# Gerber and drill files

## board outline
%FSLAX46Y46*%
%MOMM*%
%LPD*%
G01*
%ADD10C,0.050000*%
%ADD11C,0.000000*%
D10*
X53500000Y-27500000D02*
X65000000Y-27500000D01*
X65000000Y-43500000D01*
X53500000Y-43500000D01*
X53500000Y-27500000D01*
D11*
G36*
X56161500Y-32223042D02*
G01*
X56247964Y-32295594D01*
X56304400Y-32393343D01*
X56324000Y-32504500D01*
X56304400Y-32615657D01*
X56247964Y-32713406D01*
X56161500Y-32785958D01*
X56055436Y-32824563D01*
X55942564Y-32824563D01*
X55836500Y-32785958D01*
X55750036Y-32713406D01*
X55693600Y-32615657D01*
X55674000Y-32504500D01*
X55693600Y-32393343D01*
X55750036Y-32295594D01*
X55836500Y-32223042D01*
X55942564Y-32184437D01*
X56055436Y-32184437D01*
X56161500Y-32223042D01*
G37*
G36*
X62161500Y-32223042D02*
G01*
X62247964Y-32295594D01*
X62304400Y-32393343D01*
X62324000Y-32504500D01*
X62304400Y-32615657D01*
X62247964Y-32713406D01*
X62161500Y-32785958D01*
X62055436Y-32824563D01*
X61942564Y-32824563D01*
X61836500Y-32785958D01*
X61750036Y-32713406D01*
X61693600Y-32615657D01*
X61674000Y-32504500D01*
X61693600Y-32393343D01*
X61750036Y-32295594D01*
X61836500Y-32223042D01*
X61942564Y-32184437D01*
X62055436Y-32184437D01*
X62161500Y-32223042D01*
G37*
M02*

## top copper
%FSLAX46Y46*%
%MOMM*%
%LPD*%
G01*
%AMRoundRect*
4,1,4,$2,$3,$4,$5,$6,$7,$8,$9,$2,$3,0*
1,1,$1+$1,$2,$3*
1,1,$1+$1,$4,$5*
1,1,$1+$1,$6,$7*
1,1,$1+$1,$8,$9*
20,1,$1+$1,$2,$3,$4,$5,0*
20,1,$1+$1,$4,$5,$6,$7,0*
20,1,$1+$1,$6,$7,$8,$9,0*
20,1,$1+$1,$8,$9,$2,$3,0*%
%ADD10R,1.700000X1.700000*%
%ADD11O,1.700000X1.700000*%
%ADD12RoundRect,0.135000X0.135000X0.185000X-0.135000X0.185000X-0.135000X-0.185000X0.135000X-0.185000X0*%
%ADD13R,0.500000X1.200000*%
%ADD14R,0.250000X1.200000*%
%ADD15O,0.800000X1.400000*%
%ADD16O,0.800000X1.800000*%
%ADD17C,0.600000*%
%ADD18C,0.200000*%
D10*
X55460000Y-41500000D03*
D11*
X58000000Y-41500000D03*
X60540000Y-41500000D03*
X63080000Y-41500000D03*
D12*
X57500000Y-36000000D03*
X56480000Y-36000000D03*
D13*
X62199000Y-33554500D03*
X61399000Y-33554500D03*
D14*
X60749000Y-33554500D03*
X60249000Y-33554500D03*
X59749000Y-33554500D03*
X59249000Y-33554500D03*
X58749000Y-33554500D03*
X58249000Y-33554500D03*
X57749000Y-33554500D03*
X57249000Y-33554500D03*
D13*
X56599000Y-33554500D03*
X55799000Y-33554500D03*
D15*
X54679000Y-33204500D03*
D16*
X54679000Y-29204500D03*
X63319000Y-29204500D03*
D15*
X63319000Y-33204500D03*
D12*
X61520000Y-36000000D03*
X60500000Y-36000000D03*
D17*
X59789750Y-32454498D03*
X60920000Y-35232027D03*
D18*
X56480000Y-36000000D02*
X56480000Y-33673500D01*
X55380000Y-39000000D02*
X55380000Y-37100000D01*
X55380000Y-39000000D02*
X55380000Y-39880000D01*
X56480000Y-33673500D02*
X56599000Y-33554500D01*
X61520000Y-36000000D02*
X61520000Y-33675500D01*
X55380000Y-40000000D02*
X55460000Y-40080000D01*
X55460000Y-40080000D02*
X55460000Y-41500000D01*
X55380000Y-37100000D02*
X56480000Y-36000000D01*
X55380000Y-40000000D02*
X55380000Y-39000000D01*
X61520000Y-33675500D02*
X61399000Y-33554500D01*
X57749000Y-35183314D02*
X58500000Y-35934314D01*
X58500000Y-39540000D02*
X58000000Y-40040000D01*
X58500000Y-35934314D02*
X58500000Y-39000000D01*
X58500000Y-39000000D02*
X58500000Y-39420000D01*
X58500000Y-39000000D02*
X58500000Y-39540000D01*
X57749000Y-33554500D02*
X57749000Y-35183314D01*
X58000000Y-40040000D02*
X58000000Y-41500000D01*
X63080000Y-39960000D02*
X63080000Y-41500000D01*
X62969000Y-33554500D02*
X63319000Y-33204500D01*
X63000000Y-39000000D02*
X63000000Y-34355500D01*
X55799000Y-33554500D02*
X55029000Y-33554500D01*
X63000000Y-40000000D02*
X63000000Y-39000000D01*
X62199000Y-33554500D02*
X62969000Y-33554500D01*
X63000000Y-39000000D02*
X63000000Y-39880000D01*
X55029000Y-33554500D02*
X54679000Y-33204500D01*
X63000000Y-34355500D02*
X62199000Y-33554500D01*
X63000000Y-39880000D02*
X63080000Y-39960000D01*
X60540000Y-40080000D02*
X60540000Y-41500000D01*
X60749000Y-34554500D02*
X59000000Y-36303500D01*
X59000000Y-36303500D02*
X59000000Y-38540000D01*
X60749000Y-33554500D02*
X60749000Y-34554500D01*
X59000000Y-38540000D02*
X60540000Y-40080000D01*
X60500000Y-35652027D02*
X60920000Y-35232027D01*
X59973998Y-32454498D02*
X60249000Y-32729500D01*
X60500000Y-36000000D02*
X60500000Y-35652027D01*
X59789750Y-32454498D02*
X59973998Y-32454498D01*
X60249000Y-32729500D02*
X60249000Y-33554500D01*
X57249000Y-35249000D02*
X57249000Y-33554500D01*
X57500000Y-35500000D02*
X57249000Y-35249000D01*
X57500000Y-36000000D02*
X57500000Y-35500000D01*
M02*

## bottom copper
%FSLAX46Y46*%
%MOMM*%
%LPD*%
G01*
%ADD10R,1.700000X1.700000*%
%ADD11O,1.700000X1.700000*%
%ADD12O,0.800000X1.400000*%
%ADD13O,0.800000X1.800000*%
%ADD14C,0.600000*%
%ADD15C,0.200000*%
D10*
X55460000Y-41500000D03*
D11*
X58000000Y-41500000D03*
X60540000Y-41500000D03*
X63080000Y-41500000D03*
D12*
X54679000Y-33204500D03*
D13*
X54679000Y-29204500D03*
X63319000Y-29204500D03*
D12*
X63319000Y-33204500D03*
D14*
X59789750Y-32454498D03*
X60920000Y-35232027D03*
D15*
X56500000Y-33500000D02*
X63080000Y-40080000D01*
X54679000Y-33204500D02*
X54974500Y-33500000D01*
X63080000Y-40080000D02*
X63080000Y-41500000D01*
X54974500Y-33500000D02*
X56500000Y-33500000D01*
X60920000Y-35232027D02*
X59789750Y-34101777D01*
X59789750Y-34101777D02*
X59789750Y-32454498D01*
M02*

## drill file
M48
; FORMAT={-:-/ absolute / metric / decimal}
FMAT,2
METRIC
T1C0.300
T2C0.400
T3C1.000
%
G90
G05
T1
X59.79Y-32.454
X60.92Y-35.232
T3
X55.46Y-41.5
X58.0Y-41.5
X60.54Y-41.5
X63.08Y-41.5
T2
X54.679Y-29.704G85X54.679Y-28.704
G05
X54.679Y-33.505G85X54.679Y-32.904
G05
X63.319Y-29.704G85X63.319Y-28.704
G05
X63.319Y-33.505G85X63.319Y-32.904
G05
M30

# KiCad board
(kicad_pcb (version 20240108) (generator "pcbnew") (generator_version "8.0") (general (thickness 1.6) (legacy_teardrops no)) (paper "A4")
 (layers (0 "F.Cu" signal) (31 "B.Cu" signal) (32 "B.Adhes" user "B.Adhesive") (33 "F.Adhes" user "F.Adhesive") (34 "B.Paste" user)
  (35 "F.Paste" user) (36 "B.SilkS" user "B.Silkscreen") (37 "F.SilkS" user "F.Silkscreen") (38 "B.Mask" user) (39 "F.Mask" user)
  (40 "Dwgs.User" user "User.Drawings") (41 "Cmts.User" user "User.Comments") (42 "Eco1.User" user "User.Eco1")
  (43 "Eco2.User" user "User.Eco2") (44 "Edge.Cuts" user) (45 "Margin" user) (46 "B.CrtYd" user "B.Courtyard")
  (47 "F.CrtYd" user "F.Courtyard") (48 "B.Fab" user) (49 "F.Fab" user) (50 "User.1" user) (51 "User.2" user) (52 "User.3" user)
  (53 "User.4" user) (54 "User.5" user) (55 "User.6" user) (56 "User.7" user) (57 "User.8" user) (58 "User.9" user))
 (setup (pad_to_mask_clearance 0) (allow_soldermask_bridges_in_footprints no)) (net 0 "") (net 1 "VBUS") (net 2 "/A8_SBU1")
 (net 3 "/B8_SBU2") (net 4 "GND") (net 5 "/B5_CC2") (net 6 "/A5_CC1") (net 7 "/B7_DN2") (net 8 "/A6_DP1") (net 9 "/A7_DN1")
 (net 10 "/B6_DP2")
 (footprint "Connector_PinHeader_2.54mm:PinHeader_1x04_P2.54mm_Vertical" (layer "F.Cu") (at 55.46 41.5 90)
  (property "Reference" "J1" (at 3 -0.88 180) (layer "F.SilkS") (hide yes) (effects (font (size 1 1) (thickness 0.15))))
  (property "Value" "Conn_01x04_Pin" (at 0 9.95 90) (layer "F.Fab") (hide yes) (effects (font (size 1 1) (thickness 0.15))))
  (pad "1" thru_hole rect (at 0 0 90) (size 1.7 1.7) (drill 1) (layers "*.Cu" "*.Mask") (remove_unused_layers no) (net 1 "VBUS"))
  (pad "2" thru_hole oval (at 0 2.54 90) (size 1.7 1.7) (drill 1) (layers "*.Cu" "*.Mask") (remove_unused_layers no) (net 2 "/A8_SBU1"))
  (pad "3" thru_hole oval (at 0 5.08 90) (size 1.7 1.7) (drill 1) (layers "*.Cu" "*.Mask") (remove_unused_layers no) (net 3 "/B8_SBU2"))
  (pad "4" thru_hole oval (at 0 7.62 90) (size 1.7 1.7) (drill 1) (layers "*.Cu" "*.Mask") (remove_unused_layers no) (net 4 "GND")))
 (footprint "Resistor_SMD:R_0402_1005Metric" (layer "F.Cu") (at 56.99 36 180)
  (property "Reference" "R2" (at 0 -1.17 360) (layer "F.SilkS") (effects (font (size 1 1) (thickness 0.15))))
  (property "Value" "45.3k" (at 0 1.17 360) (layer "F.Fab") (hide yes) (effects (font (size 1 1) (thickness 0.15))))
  (pad "1" smd roundrect (at -0.51 0 180) (size 0.54 0.64) (layers "F.Cu" "F.Paste" "F.Mask") (roundrect_rratio 0.25) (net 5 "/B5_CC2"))
  (pad "2" smd roundrect (at 0.51 0 180) (size 0.54 0.64) (layers "F.Cu" "F.Paste" "F.Mask") (roundrect_rratio 0.25) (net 1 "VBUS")))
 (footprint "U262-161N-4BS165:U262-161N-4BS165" (layer "F.Cu") (at 58.999 31.3795 180)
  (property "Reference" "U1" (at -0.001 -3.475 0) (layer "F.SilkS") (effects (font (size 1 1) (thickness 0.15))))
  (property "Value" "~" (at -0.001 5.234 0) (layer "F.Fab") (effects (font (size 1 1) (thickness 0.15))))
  (fp_poly
   (pts (xy 3.325 -1.125) (xy 3.3054 -1.236157) (xy 3.248964 -1.333906) (xy 3.1625 -1.406458) (xy 3.056436 -1.445063)
    (xy 2.943564 -1.445063) (xy 2.8375 -1.406458) (xy 2.751036 -1.333906) (xy 2.6946 -1.236157) (xy 2.675 -1.125) (xy 2.6946 -1.013843)
    (xy 2.751036 -0.916094) (xy 2.8375 -0.843542) (xy 2.943564 -0.804937) (xy 3.056436 -0.804937) (xy 3.1625 -0.843542)
    (xy 3.248964 -0.916094) (xy 3.3054 -1.013843))
   (stroke (width 0) (type default)) (fill solid) (layer "Edge.Cuts"))
  (fp_poly
   (pts (xy -2.675 -1.125) (xy -2.6946 -1.236157) (xy -2.751036 -1.333906) (xy -2.8375 -1.406458) (xy -2.943564 -1.445063)
    (xy -3.056436 -1.445063) (xy -3.1625 -1.406458) (xy -3.248964 -1.333906) (xy -3.3054 -1.236157) (xy -3.325 -1.125)
    (xy -3.3054 -1.013843) (xy -3.248964 -0.916094) (xy -3.1625 -0.843542) (xy -3.056436 -0.804937) (xy -2.943564 -0.804937)
    (xy -2.8375 -0.843542) (xy -2.751036 -0.916094) (xy -2.6946 -1.013843))
   (stroke (width 0) (type default)) (fill solid) (layer "Edge.Cuts"))
  (pad "1" smd rect (at -3.2 -2.175 180) (size 0.5 1.2) (layers "F.Cu" "F.Paste" "F.Mask") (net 4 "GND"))
  (pad "2" smd rect (at -2.4 -2.175 180) (size 0.5 1.2) (layers "F.Cu" "F.Paste" "F.Mask") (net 1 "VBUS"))
  (pad "3" smd rect (at -1.75 -2.175 180) (size 0.25 1.2) (layers "F.Cu" "F.Paste" "F.Mask") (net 3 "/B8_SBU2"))
  (pad "4" smd rect (at -1.25 -2.175 180) (size 0.25 1.2) (layers "F.Cu" "F.Paste" "F.Mask") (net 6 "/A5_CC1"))
  (pad "5" smd rect (at -0.75 -2.175 180) (size 0.25 1.2) (layers "F.Cu" "F.Paste" "F.Mask") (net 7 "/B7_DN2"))
  (pad "6" smd rect (at -0.25 -2.175 180) (size 0.25 1.2) (layers "F.Cu" "F.Paste" "F.Mask") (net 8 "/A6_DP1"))
  (pad "7" smd rect (at 0.25 -2.175 180) (size 0.25 1.2) (layers "F.Cu" "F.Paste" "F.Mask") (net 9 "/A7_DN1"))
  (pad "8" smd rect (at 0.75 -2.175 180) (size 0.25 1.2) (layers "F.Cu" "F.Paste" "F.Mask") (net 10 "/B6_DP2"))
  (pad "9" smd rect (at 1.25 -2.175 180) (size 0.25 1.2) (layers "F.Cu" "F.Paste" "F.Mask") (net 2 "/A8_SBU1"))
  (pad "10" smd rect (at 1.75 -2.175 180) (size 0.25 1.2) (layers "F.Cu" "F.Paste" "F.Mask") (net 5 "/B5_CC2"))
  (pad "11" smd rect (at 2.4 -2.175 180) (size 0.5 1.2) (layers "F.Cu" "F.Paste" "F.Mask") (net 1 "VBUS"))
  (pad "12" smd rect (at 3.2 -2.175 180) (size 0.5 1.2) (layers "F.Cu" "F.Paste" "F.Mask") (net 4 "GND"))
  (pad "13" thru_hole oval (at 4.32 -1.825 180) (size 0.8 1.4) (drill oval 0.4 1) (layers "*.Cu" "*.Mask") (remove_unused_layers no)
   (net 4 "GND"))
  (pad "14" thru_hole oval (at 4.32 2.175 180) (size 0.8 1.8) (drill oval 0.4 1.4) (layers "*.Cu" "*.Mask") (remove_unused_layers no)
   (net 4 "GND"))
  (pad "15" thru_hole oval (at -4.32 2.175 180) (size 0.8 1.8) (drill oval 0.4 1.4) (layers "*.Cu" "*.Mask") (remove_unused_layers no)
   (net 4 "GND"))
  (pad "16" thru_hole oval (at -4.32 -1.825 180) (size 0.8 1.4) (drill oval 0.4 1) (layers "*.Cu" "*.Mask") (remove_unused_layers no)
   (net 4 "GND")))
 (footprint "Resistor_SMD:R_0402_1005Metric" (layer "F.Cu") (at 61.01 36 180)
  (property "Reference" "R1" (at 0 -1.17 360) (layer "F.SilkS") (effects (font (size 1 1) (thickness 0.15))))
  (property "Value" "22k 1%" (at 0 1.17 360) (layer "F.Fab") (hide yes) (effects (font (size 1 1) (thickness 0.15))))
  (pad "1" smd roundrect (at -0.51 0 180) (size 0.54 0.64) (layers "F.Cu" "F.Paste" "F.Mask") (roundrect_rratio 0.25) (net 1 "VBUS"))
  (pad "2" smd roundrect (at 0.51 0 180) (size 0.54 0.64) (layers "F.Cu" "F.Paste" "F.Mask") (roundrect_rratio 0.25) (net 6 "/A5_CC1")))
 (gr_rect (start 53.5 27.5) (end 65 43.5) (stroke (width 0.05) (type default)) (fill none) (layer "Edge.Cuts"))
 (segment (start 56.48 36) (end 56.48 33.6735) (width 0.2) (layer "F.Cu") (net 1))
 (segment (start 55.38 39) (end 55.38 37.1) (width 0.2) (layer "F.Cu") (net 1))
 (segment (start 55.38 39) (end 55.38 39.88) (width 0.2) (layer "F.Cu") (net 1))
 (segment (start 56.48 33.6735) (end 56.599 33.5545) (width 0.2) (layer "F.Cu") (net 1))
 (segment (start 61.52 36) (end 61.52 33.6755) (width 0.2) (layer "F.Cu") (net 1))
 (segment (start 55.38 40) (end 55.46 40.08) (width 0.2) (layer "F.Cu") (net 1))
 (segment (start 55.46 40.08) (end 55.46 41.5) (width 0.2) (layer "F.Cu") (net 1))
 (segment (start 55.38 37.1) (end 56.48 36) (width 0.2) (layer "F.Cu") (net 1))
 (segment (start 55.38 40) (end 55.38 39) (width 0.2) (layer "F.Cu") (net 1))
 (segment (start 61.52 33.6755) (end 61.399 33.5545) (width 0.2) (layer "F.Cu") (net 1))
 (segment (start 57.749 35.183314) (end 58.5 35.934314) (width 0.2) (layer "F.Cu") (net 2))
 (segment (start 58.5 39.54) (end 58 40.04) (width 0.2) (layer "F.Cu") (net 2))
 (segment (start 58.5 35.934314) (end 58.5 39) (width 0.2) (layer "F.Cu") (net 2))
 (segment (start 58.5 39) (end 58.5 39.42) (width 0.2) (layer "F.Cu") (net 2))
 (segment (start 58.5 39) (end 58.5 39.54) (width 0.2) (layer "F.Cu") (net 2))
 (segment (start 57.749 33.5545) (end 57.749 35.183314) (width 0.2) (layer "F.Cu") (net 2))
 (segment (start 58 40.04) (end 58 41.5) (width 0.2) (layer "F.Cu") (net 2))
 (segment (start 63.08 39.96) (end 63.08 41.5) (width 0.2) (layer "F.Cu") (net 4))
 (segment (start 62.969 33.5545) (end 63.319 33.2045) (width 0.2) (layer "F.Cu") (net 4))
 (segment (start 63 39) (end 63 34.3555) (width 0.2) (layer "F.Cu") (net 4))
 (segment (start 55.799 33.5545) (end 55.029 33.5545) (width 0.2) (layer "F.Cu") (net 4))
 (segment (start 63 40) (end 63 39) (width 0.2) (layer "F.Cu") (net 4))
 (segment (start 62.199 33.5545) (end 62.969 33.5545) (width 0.2) (layer "F.Cu") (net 4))
 (segment (start 63 39) (end 63 39.88) (width 0.2) (layer "F.Cu") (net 4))
 (segment (start 55.029 33.5545) (end 54.679 33.2045) (width 0.2) (layer "F.Cu") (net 4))
 (segment (start 63 34.3555) (end 62.199 33.5545) (width 0.2) (layer "F.Cu") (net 4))
 (segment (start 63 39.88) (end 63.08 39.96) (width 0.2) (layer "F.Cu") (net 4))
 (segment (start 56.5 33.5) (end 63.08 40.08) (width 0.2) (layer "B.Cu") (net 4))
 (segment (start 54.679 33.2045) (end 54.9745 33.5) (width 0.2) (layer "B.Cu") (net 4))
 (segment (start 63.08 40.08) (end 63.08 41.5) (width 0.2) (layer "B.Cu") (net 4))
 (segment (start 54.9745 33.5) (end 56.5 33.5) (width 0.2) (layer "B.Cu") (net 4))
 (segment (start 60.54 40.08) (end 60.54 41.5) (width 0.2) (layer "F.Cu") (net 3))
 (segment (start 60.749 34.5545) (end 59 36.3035) (width 0.2) (layer "F.Cu") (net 3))
 (segment (start 59 36.3035) (end 59 38.54) (width 0.2) (layer "F.Cu") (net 3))
 (segment (start 60.749 33.5545) (end 60.749 34.5545) (width 0.2) (layer "F.Cu") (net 3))
 (segment (start 59 38.54) (end 60.54 40.08) (width 0.2) (layer "F.Cu") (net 3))
 (segment (start 60.5 35.652027) (end 60.92 35.232027) (width 0.2) (layer "F.Cu") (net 6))
 (segment (start 59.973998 32.454498) (end 60.249 32.7295) (width 0.2) (layer "F.Cu") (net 6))
 (segment (start 60.5 36) (end 60.5 35.652027) (width 0.2) (layer "F.Cu") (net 6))
 (segment (start 59.78975 32.454498) (end 59.973998 32.454498) (width 0.2) (layer "F.Cu") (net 6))
 (segment (start 60.249 32.7295) (end 60.249 33.5545) (width 0.2) (layer "F.Cu") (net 6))
 (via (at 59.78975 32.454498) (size 0.6) (drill 0.3) (layers "F.Cu" "B.Cu") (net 6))
 (via (at 60.92 35.232027) (size 0.6) (drill 0.3) (layers "F.Cu" "B.Cu") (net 6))
 (segment (start 60.92 35.232027) (end 59.78975 34.101777) (width 0.2) (layer "B.Cu") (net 6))
 (segment (start 59.78975 34.101777) (end 59.78975 32.454498) (width 0.2) (layer "B.Cu") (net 6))
 (segment (start 57.249 35.249) (end 57.249 33.5545) (width 0.2) (layer "F.Cu") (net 5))
 (segment (start 57.5 35.5) (end 57.249 35.249) (width 0.2) (layer "F.Cu") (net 5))
 (segment (start 57.5 36) (end 57.5 35.5) (width 0.2) (layer "F.Cu") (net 5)))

